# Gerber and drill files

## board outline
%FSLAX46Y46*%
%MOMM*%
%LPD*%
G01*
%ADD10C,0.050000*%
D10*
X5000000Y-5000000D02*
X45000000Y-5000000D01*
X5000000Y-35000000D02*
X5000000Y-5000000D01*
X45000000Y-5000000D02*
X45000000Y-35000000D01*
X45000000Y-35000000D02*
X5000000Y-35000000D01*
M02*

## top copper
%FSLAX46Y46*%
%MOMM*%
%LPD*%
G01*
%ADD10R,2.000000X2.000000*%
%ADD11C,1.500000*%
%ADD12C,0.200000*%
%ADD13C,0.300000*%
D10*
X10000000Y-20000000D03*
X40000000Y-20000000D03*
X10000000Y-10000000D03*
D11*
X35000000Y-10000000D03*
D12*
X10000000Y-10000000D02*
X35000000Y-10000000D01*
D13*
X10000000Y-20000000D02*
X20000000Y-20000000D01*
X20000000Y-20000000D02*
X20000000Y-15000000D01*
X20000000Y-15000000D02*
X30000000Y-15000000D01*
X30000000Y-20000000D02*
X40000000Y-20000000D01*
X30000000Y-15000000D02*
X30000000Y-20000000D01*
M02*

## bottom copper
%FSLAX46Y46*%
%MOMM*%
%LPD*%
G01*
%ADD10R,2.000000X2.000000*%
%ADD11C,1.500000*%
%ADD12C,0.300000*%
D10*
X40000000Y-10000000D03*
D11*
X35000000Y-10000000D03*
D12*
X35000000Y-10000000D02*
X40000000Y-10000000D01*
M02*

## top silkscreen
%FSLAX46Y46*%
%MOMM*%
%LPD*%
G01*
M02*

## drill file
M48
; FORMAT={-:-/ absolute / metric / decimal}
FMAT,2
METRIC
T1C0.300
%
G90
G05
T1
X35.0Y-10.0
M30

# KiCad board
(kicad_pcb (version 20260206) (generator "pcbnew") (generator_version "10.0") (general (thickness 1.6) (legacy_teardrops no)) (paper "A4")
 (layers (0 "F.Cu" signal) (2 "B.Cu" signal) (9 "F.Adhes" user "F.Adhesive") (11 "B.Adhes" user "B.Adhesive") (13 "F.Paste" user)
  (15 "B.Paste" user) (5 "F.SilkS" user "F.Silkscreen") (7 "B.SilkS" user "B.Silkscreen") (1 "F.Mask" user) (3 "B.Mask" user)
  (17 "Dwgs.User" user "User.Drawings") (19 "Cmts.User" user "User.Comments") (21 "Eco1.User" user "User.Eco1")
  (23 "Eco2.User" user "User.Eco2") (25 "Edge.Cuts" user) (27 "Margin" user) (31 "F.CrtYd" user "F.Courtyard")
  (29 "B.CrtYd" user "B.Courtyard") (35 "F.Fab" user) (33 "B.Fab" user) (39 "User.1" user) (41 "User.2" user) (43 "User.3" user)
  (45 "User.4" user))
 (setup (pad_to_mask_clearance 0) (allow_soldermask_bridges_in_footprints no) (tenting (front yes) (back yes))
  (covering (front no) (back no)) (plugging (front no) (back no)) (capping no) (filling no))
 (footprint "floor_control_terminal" (layer "F.Cu") (at 10 20)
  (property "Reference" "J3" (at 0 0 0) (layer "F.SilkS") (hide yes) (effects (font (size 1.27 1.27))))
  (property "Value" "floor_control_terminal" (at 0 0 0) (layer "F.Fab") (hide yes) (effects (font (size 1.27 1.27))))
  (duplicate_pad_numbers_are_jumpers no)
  (pad "1" smd rect (at 0 0) (size 2 2) (layers "F.Cu" "F.Mask" "F.Paste") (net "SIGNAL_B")))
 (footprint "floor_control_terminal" (layer "F.Cu") (at 40 20)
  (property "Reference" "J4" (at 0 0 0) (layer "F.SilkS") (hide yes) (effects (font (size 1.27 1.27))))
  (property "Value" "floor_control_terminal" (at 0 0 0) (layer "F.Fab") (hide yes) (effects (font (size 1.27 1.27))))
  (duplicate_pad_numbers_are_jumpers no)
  (pad "1" smd rect (at 0 0) (size 2 2) (layers "F.Cu" "F.Mask" "F.Paste") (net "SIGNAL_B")))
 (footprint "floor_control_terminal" (layer "F.Cu") (at 10 10)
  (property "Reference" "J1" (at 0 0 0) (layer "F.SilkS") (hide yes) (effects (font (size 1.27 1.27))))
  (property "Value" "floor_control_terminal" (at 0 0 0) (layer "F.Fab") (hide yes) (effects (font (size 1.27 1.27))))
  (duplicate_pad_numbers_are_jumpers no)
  (pad "1" smd rect (at 0 0) (size 2 2) (layers "F.Cu" "F.Mask" "F.Paste") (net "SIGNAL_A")))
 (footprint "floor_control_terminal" (layer "B.Cu") (at 40 10)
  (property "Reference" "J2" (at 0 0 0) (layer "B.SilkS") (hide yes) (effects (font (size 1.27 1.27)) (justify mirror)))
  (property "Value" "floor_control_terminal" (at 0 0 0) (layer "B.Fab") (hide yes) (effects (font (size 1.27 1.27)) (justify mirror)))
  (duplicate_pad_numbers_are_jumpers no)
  (pad "1" smd rect (at 0 0) (size 2 2) (layers "B.Cu" "B.Mask" "B.Paste") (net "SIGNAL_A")))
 (gr_line (start 5 5) (end 45 5) (stroke (width 0.05) (type default)) (layer "Edge.Cuts"))
 (gr_line (start 5 35) (end 5 5) (stroke (width 0.05) (type default)) (layer "Edge.Cuts"))
 (gr_line (start 45 5) (end 45 35) (stroke (width 0.05) (type default)) (layer "Edge.Cuts"))
 (gr_line (start 45 35) (end 5 35) (stroke (width 0.05) (type default)) (layer "Edge.Cuts"))
 (segment (start 10 10) (end 35 10) (width 0.2) (layer "F.Cu") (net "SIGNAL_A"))
 (via (at 35 10) (size 1.5) (drill 0.3) (layers "F.Cu" "B.Cu") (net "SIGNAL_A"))
 (segment (start 35 10) (end 40 10) (width 0.3) (layer "B.Cu") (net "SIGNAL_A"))
 (segment (start 10 20) (end 20 20) (width 0.3) (layer "F.Cu") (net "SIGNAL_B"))
 (segment (start 20 20) (end 20 15) (width 0.3) (layer "F.Cu") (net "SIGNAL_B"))
 (segment (start 20 15) (end 30 15) (width 0.3) (layer "F.Cu") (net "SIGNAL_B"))
 (segment (start 30 20) (end 40 20) (width 0.3) (layer "F.Cu") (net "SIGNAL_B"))
 (segment (start 30 15) (end 30 20) (width 0.3) (layer "F.Cu") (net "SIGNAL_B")))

